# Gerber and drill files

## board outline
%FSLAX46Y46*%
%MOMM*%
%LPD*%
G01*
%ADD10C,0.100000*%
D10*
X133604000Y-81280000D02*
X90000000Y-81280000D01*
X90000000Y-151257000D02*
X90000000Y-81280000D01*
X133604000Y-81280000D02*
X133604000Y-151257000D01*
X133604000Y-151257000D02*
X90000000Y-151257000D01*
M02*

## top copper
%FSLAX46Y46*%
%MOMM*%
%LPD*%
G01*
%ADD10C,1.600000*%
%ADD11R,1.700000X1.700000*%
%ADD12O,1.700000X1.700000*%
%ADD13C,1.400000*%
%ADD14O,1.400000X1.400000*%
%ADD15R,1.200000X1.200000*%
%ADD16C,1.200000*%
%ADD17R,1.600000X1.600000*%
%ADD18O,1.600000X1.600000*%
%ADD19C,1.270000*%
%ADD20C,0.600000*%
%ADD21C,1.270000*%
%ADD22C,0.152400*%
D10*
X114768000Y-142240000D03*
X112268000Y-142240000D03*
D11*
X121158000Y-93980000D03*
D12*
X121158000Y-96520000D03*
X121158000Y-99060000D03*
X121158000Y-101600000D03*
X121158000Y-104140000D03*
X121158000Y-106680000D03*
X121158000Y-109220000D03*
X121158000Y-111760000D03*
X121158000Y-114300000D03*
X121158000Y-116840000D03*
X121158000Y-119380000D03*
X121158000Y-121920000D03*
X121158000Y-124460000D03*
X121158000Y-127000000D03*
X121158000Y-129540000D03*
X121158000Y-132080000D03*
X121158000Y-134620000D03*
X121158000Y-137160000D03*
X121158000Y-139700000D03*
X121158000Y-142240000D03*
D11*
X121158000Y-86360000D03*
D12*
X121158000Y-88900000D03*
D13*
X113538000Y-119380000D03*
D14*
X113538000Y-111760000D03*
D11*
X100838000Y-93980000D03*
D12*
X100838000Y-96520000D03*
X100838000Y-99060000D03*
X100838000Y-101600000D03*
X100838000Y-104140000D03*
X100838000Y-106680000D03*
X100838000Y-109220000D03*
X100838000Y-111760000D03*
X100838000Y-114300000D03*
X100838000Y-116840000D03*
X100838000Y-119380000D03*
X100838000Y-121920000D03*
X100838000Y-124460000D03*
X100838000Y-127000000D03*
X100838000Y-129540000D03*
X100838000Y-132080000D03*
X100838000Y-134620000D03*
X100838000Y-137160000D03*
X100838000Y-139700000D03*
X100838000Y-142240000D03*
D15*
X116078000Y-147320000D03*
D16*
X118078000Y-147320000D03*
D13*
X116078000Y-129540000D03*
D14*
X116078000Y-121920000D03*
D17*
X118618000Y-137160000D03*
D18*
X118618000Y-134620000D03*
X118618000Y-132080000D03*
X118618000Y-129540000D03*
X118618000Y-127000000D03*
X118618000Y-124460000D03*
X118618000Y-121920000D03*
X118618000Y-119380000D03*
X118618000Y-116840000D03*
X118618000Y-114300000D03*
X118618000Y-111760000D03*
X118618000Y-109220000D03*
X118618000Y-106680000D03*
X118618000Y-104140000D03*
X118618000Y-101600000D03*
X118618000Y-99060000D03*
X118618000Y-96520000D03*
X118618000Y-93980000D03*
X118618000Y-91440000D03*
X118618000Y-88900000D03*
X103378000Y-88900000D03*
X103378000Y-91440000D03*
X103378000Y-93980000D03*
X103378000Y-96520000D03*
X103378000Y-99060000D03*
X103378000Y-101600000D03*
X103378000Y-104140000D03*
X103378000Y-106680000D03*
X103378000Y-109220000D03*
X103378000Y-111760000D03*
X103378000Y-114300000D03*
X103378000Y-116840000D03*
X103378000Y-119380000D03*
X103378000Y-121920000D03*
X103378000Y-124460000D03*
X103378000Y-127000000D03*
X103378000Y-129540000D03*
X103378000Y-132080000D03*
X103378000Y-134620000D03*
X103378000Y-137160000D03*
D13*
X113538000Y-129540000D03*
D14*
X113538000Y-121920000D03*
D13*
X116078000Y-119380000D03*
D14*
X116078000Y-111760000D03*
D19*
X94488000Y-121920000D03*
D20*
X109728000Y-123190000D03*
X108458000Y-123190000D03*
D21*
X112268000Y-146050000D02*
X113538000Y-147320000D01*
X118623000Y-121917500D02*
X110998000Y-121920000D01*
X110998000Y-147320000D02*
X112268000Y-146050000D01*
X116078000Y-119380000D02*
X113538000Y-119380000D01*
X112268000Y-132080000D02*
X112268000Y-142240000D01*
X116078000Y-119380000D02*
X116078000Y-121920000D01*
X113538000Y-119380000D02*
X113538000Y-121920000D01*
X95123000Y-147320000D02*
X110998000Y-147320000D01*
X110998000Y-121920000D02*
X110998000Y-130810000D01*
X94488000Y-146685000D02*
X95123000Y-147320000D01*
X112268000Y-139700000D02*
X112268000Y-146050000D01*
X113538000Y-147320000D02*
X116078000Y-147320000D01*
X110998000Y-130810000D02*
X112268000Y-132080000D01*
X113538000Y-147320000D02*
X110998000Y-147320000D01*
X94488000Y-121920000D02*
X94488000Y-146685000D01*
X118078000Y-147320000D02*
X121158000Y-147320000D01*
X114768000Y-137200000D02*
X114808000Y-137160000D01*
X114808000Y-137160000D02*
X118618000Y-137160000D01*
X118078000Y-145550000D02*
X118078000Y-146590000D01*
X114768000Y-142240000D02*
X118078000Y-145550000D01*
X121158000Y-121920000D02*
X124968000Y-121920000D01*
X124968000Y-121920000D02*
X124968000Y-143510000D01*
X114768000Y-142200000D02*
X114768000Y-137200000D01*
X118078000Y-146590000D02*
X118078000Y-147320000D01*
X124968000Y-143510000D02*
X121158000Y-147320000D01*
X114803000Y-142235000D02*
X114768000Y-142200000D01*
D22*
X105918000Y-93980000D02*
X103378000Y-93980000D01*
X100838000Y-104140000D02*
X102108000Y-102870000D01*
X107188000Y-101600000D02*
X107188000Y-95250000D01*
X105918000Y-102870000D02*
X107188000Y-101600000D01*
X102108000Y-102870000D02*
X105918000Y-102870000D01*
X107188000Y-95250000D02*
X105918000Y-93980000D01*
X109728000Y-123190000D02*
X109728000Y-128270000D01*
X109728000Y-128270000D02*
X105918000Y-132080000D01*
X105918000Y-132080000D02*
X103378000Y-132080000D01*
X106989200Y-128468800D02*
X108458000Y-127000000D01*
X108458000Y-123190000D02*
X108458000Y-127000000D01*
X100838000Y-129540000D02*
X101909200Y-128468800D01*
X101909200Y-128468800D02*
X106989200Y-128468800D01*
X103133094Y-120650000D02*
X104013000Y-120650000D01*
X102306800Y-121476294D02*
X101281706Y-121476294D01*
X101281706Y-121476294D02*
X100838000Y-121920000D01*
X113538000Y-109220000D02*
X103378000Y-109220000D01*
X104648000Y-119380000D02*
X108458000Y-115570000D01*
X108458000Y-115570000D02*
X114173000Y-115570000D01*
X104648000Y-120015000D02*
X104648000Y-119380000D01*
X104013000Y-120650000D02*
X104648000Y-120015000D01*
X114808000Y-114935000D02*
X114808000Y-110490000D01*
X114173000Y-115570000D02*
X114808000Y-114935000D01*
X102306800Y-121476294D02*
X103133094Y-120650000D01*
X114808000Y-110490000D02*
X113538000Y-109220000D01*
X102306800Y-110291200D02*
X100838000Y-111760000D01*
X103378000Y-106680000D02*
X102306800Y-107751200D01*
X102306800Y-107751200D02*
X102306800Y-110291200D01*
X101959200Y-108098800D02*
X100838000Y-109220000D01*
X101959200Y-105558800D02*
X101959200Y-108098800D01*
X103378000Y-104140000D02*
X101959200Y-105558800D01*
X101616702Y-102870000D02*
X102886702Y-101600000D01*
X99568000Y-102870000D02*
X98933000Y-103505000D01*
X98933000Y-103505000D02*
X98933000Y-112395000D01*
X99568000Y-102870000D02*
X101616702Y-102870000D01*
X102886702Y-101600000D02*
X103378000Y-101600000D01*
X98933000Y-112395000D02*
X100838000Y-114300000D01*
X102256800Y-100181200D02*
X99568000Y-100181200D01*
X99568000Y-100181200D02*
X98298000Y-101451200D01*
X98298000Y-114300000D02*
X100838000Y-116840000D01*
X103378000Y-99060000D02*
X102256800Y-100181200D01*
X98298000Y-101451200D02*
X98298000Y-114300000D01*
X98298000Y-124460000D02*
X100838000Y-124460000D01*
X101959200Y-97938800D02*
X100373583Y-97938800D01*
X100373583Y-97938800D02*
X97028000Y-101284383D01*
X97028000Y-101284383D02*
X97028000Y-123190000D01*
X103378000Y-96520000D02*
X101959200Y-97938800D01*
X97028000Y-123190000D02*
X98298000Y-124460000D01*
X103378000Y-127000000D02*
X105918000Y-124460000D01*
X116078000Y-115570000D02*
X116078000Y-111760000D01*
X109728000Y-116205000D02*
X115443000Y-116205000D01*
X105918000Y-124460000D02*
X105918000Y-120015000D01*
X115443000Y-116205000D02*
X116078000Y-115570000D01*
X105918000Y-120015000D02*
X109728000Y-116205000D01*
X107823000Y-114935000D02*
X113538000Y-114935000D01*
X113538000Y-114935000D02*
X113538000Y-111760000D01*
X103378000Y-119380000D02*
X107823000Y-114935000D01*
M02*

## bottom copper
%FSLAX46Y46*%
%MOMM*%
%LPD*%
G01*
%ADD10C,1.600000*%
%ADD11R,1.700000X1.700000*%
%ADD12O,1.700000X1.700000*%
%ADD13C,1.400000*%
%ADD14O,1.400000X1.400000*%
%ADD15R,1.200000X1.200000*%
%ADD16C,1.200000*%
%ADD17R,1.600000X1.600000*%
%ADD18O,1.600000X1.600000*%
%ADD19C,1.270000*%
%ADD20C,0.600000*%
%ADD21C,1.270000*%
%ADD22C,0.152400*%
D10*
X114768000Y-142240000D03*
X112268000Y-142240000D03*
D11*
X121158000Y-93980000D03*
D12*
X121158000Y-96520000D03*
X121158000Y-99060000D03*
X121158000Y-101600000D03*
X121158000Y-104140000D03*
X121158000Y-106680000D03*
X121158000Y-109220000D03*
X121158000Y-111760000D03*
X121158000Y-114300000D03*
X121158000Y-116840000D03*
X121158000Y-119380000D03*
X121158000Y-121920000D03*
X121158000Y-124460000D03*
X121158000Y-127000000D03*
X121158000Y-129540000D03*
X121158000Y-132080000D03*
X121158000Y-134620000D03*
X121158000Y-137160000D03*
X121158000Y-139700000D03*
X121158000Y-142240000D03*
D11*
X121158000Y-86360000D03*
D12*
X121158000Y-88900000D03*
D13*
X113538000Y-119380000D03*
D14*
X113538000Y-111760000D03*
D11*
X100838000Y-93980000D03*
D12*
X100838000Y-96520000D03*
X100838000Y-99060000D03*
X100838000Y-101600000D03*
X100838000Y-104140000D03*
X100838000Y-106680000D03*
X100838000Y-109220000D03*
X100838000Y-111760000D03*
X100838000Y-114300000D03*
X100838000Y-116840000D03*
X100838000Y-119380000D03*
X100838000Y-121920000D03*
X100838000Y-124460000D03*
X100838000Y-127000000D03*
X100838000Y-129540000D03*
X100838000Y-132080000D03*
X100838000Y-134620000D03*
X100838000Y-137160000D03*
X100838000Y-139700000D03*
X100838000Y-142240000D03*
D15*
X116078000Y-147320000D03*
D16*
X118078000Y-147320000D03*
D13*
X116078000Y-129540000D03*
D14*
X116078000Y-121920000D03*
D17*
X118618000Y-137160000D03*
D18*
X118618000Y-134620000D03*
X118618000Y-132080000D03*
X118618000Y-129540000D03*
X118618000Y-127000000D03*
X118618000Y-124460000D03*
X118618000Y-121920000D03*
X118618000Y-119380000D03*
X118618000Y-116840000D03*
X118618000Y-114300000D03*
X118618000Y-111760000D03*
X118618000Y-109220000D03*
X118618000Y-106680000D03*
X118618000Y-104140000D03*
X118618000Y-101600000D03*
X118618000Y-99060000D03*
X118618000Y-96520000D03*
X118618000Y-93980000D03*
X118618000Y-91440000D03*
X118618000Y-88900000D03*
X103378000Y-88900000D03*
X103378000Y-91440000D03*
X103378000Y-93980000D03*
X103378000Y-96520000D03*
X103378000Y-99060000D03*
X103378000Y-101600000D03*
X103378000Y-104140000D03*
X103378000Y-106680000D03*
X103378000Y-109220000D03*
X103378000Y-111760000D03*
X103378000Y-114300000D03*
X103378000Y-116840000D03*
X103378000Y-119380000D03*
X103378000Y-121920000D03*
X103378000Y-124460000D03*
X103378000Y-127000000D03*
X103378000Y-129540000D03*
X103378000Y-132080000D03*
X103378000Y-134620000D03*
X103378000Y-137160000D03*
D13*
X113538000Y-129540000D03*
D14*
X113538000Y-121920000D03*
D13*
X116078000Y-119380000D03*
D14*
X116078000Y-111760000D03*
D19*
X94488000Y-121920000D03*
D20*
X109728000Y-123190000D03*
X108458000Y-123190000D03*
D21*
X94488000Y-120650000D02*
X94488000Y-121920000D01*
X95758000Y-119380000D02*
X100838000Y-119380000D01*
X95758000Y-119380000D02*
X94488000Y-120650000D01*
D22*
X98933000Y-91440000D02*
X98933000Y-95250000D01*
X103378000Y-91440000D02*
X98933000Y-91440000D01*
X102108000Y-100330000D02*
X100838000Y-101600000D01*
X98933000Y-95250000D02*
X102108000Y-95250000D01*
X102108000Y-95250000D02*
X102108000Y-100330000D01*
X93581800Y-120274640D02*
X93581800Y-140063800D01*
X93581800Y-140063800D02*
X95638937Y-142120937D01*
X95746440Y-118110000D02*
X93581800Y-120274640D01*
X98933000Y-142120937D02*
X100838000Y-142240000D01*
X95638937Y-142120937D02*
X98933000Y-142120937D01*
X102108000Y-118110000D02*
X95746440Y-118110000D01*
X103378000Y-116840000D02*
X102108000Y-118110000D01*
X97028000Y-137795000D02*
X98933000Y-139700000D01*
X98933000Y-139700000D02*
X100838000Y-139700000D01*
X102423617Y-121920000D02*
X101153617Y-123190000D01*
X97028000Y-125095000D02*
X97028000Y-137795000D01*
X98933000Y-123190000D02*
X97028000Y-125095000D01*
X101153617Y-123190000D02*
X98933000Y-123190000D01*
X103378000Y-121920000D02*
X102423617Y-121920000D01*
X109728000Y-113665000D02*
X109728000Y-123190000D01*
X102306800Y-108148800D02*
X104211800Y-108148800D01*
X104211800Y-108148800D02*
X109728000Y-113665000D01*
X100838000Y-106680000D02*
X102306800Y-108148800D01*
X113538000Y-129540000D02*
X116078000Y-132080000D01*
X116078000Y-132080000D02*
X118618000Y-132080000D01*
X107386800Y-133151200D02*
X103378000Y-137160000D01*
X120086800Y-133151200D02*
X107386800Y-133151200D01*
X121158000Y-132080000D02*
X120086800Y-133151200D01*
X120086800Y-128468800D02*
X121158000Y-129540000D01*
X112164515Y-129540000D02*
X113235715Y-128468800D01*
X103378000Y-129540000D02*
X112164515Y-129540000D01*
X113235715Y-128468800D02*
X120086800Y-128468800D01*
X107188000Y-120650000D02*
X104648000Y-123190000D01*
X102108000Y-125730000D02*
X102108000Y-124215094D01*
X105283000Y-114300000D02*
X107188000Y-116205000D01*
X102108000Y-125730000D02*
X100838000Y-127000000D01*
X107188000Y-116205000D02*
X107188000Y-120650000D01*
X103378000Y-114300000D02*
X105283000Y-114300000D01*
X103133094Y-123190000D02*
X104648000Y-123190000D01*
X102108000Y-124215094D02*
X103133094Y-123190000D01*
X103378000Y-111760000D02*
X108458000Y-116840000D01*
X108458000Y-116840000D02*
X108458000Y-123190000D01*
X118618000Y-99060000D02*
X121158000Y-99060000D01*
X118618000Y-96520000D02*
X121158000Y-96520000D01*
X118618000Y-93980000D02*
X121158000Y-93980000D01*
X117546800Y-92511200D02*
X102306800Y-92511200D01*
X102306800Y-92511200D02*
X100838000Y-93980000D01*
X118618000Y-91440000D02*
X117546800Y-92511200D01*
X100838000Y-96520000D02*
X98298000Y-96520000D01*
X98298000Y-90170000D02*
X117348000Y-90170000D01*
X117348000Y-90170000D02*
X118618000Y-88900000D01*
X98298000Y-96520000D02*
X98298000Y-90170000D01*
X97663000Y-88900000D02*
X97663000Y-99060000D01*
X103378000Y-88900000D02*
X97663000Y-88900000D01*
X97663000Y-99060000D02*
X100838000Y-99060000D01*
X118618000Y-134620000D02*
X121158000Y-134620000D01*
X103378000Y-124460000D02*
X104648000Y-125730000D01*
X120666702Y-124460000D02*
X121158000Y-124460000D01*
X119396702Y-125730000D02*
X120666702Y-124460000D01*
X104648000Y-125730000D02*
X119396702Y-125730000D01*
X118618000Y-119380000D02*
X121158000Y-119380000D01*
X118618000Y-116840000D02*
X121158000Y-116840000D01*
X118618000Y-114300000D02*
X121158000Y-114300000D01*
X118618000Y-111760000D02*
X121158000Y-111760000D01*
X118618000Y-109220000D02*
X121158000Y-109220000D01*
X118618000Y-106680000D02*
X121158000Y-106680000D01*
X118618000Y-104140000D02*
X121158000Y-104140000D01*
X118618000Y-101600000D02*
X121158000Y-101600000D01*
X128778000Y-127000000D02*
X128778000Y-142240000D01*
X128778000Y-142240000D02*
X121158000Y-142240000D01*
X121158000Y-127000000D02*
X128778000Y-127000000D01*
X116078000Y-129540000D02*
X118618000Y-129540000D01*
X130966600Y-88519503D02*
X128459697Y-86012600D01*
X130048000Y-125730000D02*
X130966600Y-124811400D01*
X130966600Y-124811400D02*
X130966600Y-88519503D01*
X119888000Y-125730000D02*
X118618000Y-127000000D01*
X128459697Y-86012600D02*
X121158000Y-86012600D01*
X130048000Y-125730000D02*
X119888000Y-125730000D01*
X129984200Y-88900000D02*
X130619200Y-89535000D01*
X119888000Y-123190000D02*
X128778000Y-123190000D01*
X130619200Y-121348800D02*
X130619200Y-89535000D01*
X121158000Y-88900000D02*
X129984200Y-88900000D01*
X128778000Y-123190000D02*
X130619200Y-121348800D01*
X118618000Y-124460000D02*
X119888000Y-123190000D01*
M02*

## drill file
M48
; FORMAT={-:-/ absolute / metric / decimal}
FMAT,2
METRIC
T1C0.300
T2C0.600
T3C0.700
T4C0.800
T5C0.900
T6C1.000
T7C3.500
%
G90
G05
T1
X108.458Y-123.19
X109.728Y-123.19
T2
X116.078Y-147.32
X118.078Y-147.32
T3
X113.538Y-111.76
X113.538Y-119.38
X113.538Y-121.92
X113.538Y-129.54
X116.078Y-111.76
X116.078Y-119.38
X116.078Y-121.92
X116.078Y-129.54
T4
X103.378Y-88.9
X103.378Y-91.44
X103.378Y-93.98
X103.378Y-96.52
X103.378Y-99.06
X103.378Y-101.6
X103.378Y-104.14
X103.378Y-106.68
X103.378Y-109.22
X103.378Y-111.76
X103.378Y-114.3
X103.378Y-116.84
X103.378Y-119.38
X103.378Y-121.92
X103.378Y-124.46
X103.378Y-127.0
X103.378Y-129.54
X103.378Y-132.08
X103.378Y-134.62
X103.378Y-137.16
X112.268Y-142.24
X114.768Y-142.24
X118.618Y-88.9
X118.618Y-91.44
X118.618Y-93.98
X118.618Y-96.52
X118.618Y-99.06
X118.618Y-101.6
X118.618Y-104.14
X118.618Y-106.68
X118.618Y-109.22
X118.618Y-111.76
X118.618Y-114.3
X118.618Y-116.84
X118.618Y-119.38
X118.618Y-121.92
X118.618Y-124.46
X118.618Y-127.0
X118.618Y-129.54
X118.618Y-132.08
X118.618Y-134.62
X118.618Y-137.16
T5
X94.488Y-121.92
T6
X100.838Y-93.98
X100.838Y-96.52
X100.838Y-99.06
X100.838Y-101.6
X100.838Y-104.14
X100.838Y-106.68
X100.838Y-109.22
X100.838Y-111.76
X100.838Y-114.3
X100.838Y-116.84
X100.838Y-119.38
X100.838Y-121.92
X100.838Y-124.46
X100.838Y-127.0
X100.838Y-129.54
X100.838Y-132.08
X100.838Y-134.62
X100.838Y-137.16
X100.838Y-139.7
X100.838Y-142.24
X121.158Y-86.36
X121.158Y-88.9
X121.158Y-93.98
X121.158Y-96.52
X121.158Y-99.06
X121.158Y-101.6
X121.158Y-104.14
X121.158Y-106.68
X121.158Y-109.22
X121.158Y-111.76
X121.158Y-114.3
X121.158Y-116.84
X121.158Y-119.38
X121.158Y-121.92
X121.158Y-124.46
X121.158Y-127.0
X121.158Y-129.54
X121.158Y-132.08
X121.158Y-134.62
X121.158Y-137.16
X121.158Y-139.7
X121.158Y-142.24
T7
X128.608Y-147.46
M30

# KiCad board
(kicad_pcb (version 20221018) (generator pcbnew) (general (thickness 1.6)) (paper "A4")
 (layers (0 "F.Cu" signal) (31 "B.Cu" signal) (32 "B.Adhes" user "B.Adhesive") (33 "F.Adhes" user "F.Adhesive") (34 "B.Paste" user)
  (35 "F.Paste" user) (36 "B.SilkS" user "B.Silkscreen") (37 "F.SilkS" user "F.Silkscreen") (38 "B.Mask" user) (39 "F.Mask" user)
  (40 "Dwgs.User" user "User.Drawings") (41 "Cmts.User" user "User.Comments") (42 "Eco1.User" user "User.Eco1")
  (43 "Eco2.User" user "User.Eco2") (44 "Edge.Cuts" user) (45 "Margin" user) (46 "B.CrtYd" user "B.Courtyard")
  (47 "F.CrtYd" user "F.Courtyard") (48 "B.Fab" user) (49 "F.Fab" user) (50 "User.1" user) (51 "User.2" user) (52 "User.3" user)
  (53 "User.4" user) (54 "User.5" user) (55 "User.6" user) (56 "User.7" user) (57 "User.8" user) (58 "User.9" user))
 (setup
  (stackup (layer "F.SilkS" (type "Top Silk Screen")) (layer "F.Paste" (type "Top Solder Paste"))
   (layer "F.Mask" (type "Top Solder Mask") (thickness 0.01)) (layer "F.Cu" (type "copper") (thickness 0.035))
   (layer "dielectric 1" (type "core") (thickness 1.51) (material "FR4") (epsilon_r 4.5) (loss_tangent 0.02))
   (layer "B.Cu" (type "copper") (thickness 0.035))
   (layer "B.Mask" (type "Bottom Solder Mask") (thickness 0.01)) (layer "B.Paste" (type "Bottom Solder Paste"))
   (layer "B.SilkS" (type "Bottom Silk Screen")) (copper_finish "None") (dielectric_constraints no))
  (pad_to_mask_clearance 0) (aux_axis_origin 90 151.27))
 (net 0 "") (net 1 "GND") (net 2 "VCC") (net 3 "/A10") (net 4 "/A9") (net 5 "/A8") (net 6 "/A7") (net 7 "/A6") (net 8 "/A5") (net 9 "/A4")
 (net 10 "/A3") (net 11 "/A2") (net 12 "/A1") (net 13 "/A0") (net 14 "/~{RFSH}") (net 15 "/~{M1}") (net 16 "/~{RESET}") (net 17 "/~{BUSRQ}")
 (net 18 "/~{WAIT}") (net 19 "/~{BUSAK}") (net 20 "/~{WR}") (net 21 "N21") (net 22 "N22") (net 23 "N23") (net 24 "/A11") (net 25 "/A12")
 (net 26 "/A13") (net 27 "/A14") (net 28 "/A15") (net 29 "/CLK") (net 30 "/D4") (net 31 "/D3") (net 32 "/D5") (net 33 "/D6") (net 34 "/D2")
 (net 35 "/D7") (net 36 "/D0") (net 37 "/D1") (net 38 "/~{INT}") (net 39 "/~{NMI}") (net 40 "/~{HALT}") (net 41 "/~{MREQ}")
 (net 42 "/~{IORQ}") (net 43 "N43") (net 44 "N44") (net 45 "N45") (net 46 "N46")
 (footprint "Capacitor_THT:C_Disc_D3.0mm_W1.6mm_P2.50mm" (layer "F.Cu") (at 114.768 142.24 180)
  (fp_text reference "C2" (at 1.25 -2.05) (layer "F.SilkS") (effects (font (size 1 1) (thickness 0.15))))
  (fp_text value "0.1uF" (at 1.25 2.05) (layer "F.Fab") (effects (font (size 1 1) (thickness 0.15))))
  (pad "1" thru_hole circle (at 0 0 180) (size 1.6 1.6) (drill 0.8) (layers "*.Cu" "*.Mask") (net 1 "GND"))
  (pad "2" thru_hole circle (at 2.5 0 180) (size 1.6 1.6) (drill 0.8) (layers "*.Cu" "*.Mask") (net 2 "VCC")))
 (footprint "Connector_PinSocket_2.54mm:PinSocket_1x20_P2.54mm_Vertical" (layer "F.Cu") (at 121.158 93.98)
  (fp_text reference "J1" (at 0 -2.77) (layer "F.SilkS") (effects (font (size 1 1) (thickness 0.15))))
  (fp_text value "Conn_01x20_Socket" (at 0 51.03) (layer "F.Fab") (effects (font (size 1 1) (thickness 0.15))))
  (pad "1" thru_hole rect (at 0 0) (size 1.7 1.7) (drill 1) (layers "*.Cu" "*.Mask") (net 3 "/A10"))
  (pad "2" thru_hole oval (at 0 2.54) (size 1.7 1.7) (drill 1) (layers "*.Cu" "*.Mask") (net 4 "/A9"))
  (pad "3" thru_hole oval (at 0 5.08) (size 1.7 1.7) (drill 1) (layers "*.Cu" "*.Mask") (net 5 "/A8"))
  (pad "4" thru_hole oval (at 0 7.62) (size 1.7 1.7) (drill 1) (layers "*.Cu" "*.Mask") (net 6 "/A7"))
  (pad "5" thru_hole oval (at 0 10.16) (size 1.7 1.7) (drill 1) (layers "*.Cu" "*.Mask") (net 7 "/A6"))
  (pad "6" thru_hole oval (at 0 12.7) (size 1.7 1.7) (drill 1) (layers "*.Cu" "*.Mask") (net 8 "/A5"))
  (pad "7" thru_hole oval (at 0 15.24) (size 1.7 1.7) (drill 1) (layers "*.Cu" "*.Mask") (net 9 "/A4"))
  (pad "8" thru_hole oval (at 0 17.78) (size 1.7 1.7) (drill 1) (layers "*.Cu" "*.Mask") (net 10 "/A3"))
  (pad "9" thru_hole oval (at 0 20.32) (size 1.7 1.7) (drill 1) (layers "*.Cu" "*.Mask") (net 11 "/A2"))
  (pad "10" thru_hole oval (at 0 22.86) (size 1.7 1.7) (drill 1) (layers "*.Cu" "*.Mask") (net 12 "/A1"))
  (pad "11" thru_hole oval (at 0 25.4) (size 1.7 1.7) (drill 1) (layers "*.Cu" "*.Mask") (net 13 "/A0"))
  (pad "12" thru_hole oval (at 0 27.94) (size 1.7 1.7) (drill 1) (layers "*.Cu" "*.Mask") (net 1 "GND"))
  (pad "13" thru_hole oval (at 0 30.48) (size 1.7 1.7) (drill 1) (layers "*.Cu" "*.Mask") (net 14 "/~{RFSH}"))
  (pad "14" thru_hole oval (at 0 33.02) (size 1.7 1.7) (drill 1) (layers "*.Cu" "*.Mask") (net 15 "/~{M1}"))
  (pad "15" thru_hole oval (at 0 35.56) (size 1.7 1.7) (drill 1) (layers "*.Cu" "*.Mask") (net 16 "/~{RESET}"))
  (pad "16" thru_hole oval (at 0 38.1) (size 1.7 1.7) (drill 1) (layers "*.Cu" "*.Mask") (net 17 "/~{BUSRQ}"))
  (pad "17" thru_hole oval (at 0 40.64) (size 1.7 1.7) (drill 1) (layers "*.Cu" "*.Mask") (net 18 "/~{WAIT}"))
  (pad "18" thru_hole oval (at 0 43.18) (size 1.7 1.7) (drill 1) (layers "*.Cu" "*.Mask") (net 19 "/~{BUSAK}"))
  (pad "19" thru_hole oval (at 0 45.72) (size 1.7 1.7) (drill 1) (layers "*.Cu" "*.Mask") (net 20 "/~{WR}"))
  (pad "20" thru_hole oval (at 0 48.26) (size 1.7 1.7) (drill 1) (layers "*.Cu" "*.Mask") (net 15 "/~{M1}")))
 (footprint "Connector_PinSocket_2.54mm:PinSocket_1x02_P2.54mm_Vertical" (layer "F.Cu") (at 121.158 86.36)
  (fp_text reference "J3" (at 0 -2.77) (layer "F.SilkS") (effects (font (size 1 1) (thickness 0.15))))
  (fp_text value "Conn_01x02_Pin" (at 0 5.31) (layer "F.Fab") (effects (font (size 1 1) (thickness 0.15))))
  (pad "1" thru_hole rect (at 0 0) (size 1.7 1.7) (drill 1) (layers "*.Cu" "*.Mask") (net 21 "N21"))
  (pad "2" thru_hole oval (at 0 2.54) (size 1.7 1.7) (drill 1) (layers "*.Cu" "*.Mask") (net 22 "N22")))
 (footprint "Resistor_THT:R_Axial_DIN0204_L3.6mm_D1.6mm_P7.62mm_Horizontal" (layer "F.Cu") (at 113.538 119.38 90)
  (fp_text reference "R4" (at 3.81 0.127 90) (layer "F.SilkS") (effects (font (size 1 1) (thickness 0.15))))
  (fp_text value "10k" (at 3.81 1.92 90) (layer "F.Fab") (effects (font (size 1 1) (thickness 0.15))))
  (pad "1" thru_hole circle (at 0 0 90) (size 1.4 1.4) (drill 0.7) (layers "*.Cu" "*.Mask") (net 2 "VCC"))
  (pad "2" thru_hole oval (at 7.62 0 90) (size 1.4 1.4) (drill 0.7) (layers "*.Cu" "*.Mask") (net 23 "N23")))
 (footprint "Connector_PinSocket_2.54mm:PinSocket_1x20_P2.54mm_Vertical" (layer "F.Cu") (at 100.838 93.98)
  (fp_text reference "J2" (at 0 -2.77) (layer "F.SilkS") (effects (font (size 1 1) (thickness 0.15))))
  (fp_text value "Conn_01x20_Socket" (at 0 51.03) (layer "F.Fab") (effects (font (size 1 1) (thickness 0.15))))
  (pad "1" thru_hole rect (at 0 0) (size 1.7 1.7) (drill 1) (layers "*.Cu" "*.Mask") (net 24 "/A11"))
  (pad "2" thru_hole oval (at 0 2.54) (size 1.7 1.7) (drill 1) (layers "*.Cu" "*.Mask") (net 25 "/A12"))
  (pad "3" thru_hole oval (at 0 5.08) (size 1.7 1.7) (drill 1) (layers "*.Cu" "*.Mask") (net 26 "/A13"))
  (pad "4" thru_hole oval (at 0 7.62) (size 1.7 1.7) (drill 1) (layers "*.Cu" "*.Mask") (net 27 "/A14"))
  (pad "5" thru_hole oval (at 0 10.16) (size 1.7 1.7) (drill 1) (layers "*.Cu" "*.Mask") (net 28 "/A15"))
  (pad "6" thru_hole oval (at 0 12.7) (size 1.7 1.7) (drill 1) (layers "*.Cu" "*.Mask") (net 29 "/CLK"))
  (pad "7" thru_hole oval (at 0 15.24) (size 1.7 1.7) (drill 1) (layers "*.Cu" "*.Mask") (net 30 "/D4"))
  (pad "8" thru_hole oval (at 0 17.78) (size 1.7 1.7) (drill 1) (layers "*.Cu" "*.Mask") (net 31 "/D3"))
  (pad "9" thru_hole oval (at 0 20.32) (size 1.7 1.7) (drill 1) (layers "*.Cu" "*.Mask") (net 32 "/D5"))
  (pad "10" thru_hole oval (at 0 22.86) (size 1.7 1.7) (drill 1) (layers "*.Cu" "*.Mask") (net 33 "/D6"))
  (pad "11" thru_hole oval (at 0 25.4) (size 1.7 1.7) (drill 1) (layers "*.Cu" "*.Mask") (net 2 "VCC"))
  (pad "12" thru_hole oval (at 0 27.94) (size 1.7 1.7) (drill 1) (layers "*.Cu" "*.Mask") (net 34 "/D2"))
  (pad "13" thru_hole oval (at 0 30.48) (size 1.7 1.7) (drill 1) (layers "*.Cu" "*.Mask") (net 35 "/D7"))
  (pad "14" thru_hole oval (at 0 33.02) (size 1.7 1.7) (drill 1) (layers "*.Cu" "*.Mask") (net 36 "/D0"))
  (pad "15" thru_hole oval (at 0 35.56) (size 1.7 1.7) (drill 1) (layers "*.Cu" "*.Mask") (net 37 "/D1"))
  (pad "16" thru_hole oval (at 0 38.1) (size 1.7 1.7) (drill 1) (layers "*.Cu" "*.Mask") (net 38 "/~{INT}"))
  (pad "17" thru_hole oval (at 0 40.64) (size 1.7 1.7) (drill 1) (layers "*.Cu" "*.Mask") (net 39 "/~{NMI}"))
  (pad "18" thru_hole oval (at 0 43.18) (size 1.7 1.7) (drill 1) (layers "*.Cu" "*.Mask") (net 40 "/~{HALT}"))
  (pad "19" thru_hole oval (at 0 45.72) (size 1.7 1.7) (drill 1) (layers "*.Cu" "*.Mask") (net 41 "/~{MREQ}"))
  (pad "20" thru_hole oval (at 0 48.26) (size 1.7 1.7) (drill 1) (layers "*.Cu" "*.Mask") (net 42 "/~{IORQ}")))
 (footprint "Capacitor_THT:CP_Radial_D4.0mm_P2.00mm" (layer "F.Cu") (at 116.078 147.32)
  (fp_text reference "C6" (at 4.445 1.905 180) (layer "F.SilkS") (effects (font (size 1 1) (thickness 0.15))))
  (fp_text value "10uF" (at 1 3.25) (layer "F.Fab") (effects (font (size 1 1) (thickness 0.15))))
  (pad "1" thru_hole rect (at 0 0) (size 1.2 1.2) (drill 0.6) (layers "*.Cu" "*.Mask") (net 2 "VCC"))
  (pad "2" thru_hole circle (at 2 0) (size 1.2 1.2) (drill 0.6) (layers "*.Cu" "*.Mask") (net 1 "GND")))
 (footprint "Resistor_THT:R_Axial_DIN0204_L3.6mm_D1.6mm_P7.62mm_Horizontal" (layer "F.Cu") (at 116.078 129.54 90)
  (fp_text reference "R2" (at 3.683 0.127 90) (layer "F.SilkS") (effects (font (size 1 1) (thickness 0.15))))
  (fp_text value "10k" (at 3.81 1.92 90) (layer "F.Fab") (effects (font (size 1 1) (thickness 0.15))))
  (pad "1" thru_hole circle (at 0 0 90) (size 1.4 1.4) (drill 0.7) (layers "*.Cu" "*.Mask") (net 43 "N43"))
  (pad "2" thru_hole oval (at 7.62 0 90) (size 1.4 1.4) (drill 0.7) (layers "*.Cu" "*.Mask") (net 2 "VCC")))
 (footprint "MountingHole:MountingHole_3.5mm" (layer "F.Cu") (at 128.608 147.46)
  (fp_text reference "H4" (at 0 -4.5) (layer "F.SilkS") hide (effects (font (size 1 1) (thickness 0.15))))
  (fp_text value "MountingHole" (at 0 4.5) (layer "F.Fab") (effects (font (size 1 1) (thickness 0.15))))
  (pad "" np_thru_hole circle (at 0 0) (size 3.5 3.5) (drill 3.5) (layers "*.Cu" "*.Mask")))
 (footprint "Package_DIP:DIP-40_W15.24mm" (layer "F.Cu") (at 118.618 137.16 180)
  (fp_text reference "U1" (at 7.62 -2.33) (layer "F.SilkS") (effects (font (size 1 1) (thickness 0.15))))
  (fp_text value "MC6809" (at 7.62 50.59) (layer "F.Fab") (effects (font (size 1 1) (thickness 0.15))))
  (pad "1" thru_hole rect (at 0 0 180) (size 1.6 1.6) (drill 0.8) (layers "*.Cu" "*.Mask") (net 1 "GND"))
  (pad "2" thru_hole oval (at 0 2.54 180) (size 1.6 1.6) (drill 0.8) (layers "*.Cu" "*.Mask") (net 18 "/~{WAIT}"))
  (pad "3" thru_hole oval (at 0 5.08 180) (size 1.6 1.6) (drill 0.8) (layers "*.Cu" "*.Mask") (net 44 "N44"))
  (pad "4" thru_hole oval (at 0 7.62 180) (size 1.6 1.6) (drill 0.8) (layers "*.Cu" "*.Mask") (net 43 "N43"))
  (pad "5" thru_hole oval (at 0 10.16 180) (size 1.6 1.6) (drill 0.8) (layers "*.Cu" "*.Mask") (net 21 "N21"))
  (pad "6" thru_hole oval (at 0 12.7 180) (size 1.6 1.6) (drill 0.8) (layers "*.Cu" "*.Mask") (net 22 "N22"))
  (pad "7" thru_hole oval (at 0 15.24 180) (size 1.6 1.6) (drill 0.8) (layers "*.Cu" "*.Mask") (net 2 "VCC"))
  (pad "8" thru_hole oval (at 0 17.78 180) (size 1.6 1.6) (drill 0.8) (layers "*.Cu" "*.Mask") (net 13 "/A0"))
  (pad "9" thru_hole oval (at 0 20.32 180) (size 1.6 1.6) (drill 0.8) (layers "*.Cu" "*.Mask") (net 12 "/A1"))
  (pad "10" thru_hole oval (at 0 22.86 180) (size 1.6 1.6) (drill 0.8) (layers "*.Cu" "*.Mask") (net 11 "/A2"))
  (pad "11" thru_hole oval (at 0 25.4 180) (size 1.6 1.6) (drill 0.8) (layers "*.Cu" "*.Mask") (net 10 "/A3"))
  (pad "12" thru_hole oval (at 0 27.94 180) (size 1.6 1.6) (drill 0.8) (layers "*.Cu" "*.Mask") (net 9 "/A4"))
  (pad "13" thru_hole oval (at 0 30.48 180) (size 1.6 1.6) (drill 0.8) (layers "*.Cu" "*.Mask") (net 8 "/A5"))
  (pad "14" thru_hole oval (at 0 33.02 180) (size 1.6 1.6) (drill 0.8) (layers "*.Cu" "*.Mask") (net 7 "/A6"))
  (pad "15" thru_hole oval (at 0 35.56 180) (size 1.6 1.6) (drill 0.8) (layers "*.Cu" "*.Mask") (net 6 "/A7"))
  (pad "16" thru_hole oval (at 0 38.1 180) (size 1.6 1.6) (drill 0.8) (layers "*.Cu" "*.Mask") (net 5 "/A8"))
  (pad "17" thru_hole oval (at 0 40.64 180) (size 1.6 1.6) (drill 0.8) (layers "*.Cu" "*.Mask") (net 4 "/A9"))
  (pad "18" thru_hole oval (at 0 43.18 180) (size 1.6 1.6) (drill 0.8) (layers "*.Cu" "*.Mask") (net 3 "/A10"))
  (pad "19" thru_hole oval (at 0 45.72 180) (size 1.6 1.6) (drill 0.8) (layers "*.Cu" "*.Mask") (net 24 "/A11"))
  (pad "20" thru_hole oval (at 0 48.26 180) (size 1.6 1.6) (drill 0.8) (layers "*.Cu" "*.Mask") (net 25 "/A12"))
  (pad "21" thru_hole oval (at 15.24 48.26 180) (size 1.6 1.6) (drill 0.8) (layers "*.Cu" "*.Mask") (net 26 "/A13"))
  (pad "22" thru_hole oval (at 15.24 45.72 180) (size 1.6 1.6) (drill 0.8) (layers "*.Cu" "*.Mask") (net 27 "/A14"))
  (pad "23" thru_hole oval (at 15.24 43.18 180) (size 1.6 1.6) (drill 0.8) (layers "*.Cu" "*.Mask") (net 28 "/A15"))
  (pad "24" thru_hole oval (at 15.24 40.64 180) (size 1.6 1.6) (drill 0.8) (layers "*.Cu" "*.Mask") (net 35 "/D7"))
  (pad "25" thru_hole oval (at 15.24 38.1 180) (size 1.6 1.6) (drill 0.8) (layers "*.Cu" "*.Mask") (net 33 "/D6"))
  (pad "26" thru_hole oval (at 15.24 35.56 180) (size 1.6 1.6) (drill 0.8) (layers "*.Cu" "*.Mask") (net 32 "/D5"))
  (pad "27" thru_hole oval (at 15.24 33.02 180) (size 1.6 1.6) (drill 0.8) (layers "*.Cu" "*.Mask") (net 30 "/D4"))
  (pad "28" thru_hole oval (at 15.24 30.48 180) (size 1.6 1.6) (drill 0.8) (layers "*.Cu" "*.Mask") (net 31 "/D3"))
  (pad "29" thru_hole oval (at 15.24 27.94 180) (size 1.6 1.6) (drill 0.8) (layers "*.Cu" "*.Mask") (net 34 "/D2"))
  (pad "30" thru_hole oval (at 15.24 25.4 180) (size 1.6 1.6) (drill 0.8) (layers "*.Cu" "*.Mask") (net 37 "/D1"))
  (pad "31" thru_hole oval (at 15.24 22.86 180) (size 1.6 1.6) (drill 0.8) (layers "*.Cu" "*.Mask") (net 36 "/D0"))
  (pad "32" thru_hole oval (at 15.24 20.32 180) (size 1.6 1.6) (drill 0.8) (layers "*.Cu" "*.Mask") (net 42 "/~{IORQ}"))
  (pad "33" thru_hole oval (at 15.24 17.78 180) (size 1.6 1.6) (drill 0.8) (layers "*.Cu" "*.Mask") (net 23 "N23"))
  (pad "34" thru_hole oval (at 15.24 15.24 180) (size 1.6 1.6) (drill 0.8) (layers "*.Cu" "*.Mask") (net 41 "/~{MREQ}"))
  (pad "35" thru_hole oval (at 15.24 12.7 180) (size 1.6 1.6) (drill 0.8) (layers "*.Cu" "*.Mask") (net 14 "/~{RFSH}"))
  (pad "36" thru_hole oval (at 15.24 10.16 180) (size 1.6 1.6) (drill 0.8) (layers "*.Cu" "*.Mask") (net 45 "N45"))
  (pad "37" thru_hole oval (at 15.24 7.62 180) (size 1.6 1.6) (drill 0.8) (layers "*.Cu" "*.Mask") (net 16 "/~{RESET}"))
  (pad "38" thru_hole oval (at 15.24 5.08 180) (size 1.6 1.6) (drill 0.8) (layers "*.Cu" "*.Mask") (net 29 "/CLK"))
  (pad "39" thru_hole oval (at 15.24 2.54 180) (size 1.6 1.6) (drill 0.8) (layers "*.Cu" "*.Mask") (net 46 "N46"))
  (pad "40" thru_hole oval (at 15.24 0 180) (size 1.6 1.6) (drill 0.8) (layers "*.Cu" "*.Mask") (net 17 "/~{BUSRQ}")))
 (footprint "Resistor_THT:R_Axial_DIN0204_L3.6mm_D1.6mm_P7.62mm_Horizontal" (layer "F.Cu") (at 113.538 129.54 90)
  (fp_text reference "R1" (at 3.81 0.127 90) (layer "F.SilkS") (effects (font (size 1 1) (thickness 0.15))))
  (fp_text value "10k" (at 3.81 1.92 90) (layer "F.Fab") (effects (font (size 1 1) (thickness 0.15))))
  (pad "1" thru_hole circle (at 0 0 90) (size 1.4 1.4) (drill 0.7) (layers "*.Cu" "*.Mask") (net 44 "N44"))
  (pad "2" thru_hole oval (at 7.62 0 90) (size 1.4 1.4) (drill 0.7) (layers "*.Cu" "*.Mask") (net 2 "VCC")))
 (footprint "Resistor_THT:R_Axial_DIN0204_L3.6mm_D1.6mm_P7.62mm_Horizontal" (layer "F.Cu") (at 116.078 119.38 90)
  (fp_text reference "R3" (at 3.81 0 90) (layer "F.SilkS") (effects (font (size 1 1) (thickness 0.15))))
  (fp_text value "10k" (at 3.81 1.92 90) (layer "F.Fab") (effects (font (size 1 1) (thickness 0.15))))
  (pad "1" thru_hole circle (at 0 0 90) (size 1.4 1.4) (drill 0.7) (layers "*.Cu" "*.Mask") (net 2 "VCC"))
  (pad "2" thru_hole oval (at 7.62 0 90) (size 1.4 1.4) (drill 0.7) (layers "*.Cu" "*.Mask") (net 45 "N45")))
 (gr_line (start 133.604 81.28) (end 90 81.28) (stroke (width 0.1) (type solid)) (layer "Edge.Cuts"))
 (gr_line (start 90 151.257) (end 90 81.28) (stroke (width 0.1) (type solid)) (layer "Edge.Cuts"))
 (gr_line (start 133.604 81.28) (end 133.604 151.257) (stroke (width 0.1) (type solid)) (layer "Edge.Cuts"))
 (gr_line (start 133.604 151.257) (end 90 151.257) (stroke (width 0.1) (type solid)) (layer "Edge.Cuts"))
 (segment (start 112.268 146.05) (end 113.538 147.32) (width 1.27) (layer "F.Cu") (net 2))
 (segment (start 118.623 121.9175) (end 110.998 121.92) (width 1.27) (layer "F.Cu") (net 2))
 (segment (start 110.998 147.32) (end 112.268 146.05) (width 1.27) (layer "F.Cu") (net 2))
 (segment (start 116.078 119.38) (end 113.538 119.38) (width 1.27) (layer "F.Cu") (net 2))
 (segment (start 112.268 132.08) (end 112.268 142.24) (width 1.27) (layer "F.Cu") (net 2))
 (segment (start 116.078 119.38) (end 116.078 121.92) (width 1.27) (layer "F.Cu") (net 2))
 (segment (start 113.538 119.38) (end 113.538 121.92) (width 1.27) (layer "F.Cu") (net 2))
 (segment (start 95.123 147.32) (end 110.998 147.32) (width 1.27) (layer "F.Cu") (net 2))
 (segment (start 110.998 121.92) (end 110.998 130.81) (width 1.27) (layer "F.Cu") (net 2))
 (segment (start 94.488 146.685) (end 95.123 147.32) (width 1.27) (layer "F.Cu") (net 2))
 (segment (start 112.268 139.7) (end 112.268 146.05) (width 1.27) (layer "F.Cu") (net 2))
 (segment (start 113.538 147.32) (end 116.078 147.32) (width 1.27) (layer "F.Cu") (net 2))
 (segment (start 110.998 130.81) (end 112.268 132.08) (width 1.27) (layer "F.Cu") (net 2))
 (segment (start 113.538 147.32) (end 110.998 147.32) (width 1.27) (layer "F.Cu") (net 2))
 (segment (start 94.488 121.92) (end 94.488 146.685) (width 1.27) (layer "F.Cu") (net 2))
 (via (at 94.488 121.92) (size 1.27) (drill 0.9) (layers "F.Cu" "B.Cu") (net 2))
 (segment (start 94.488 120.65) (end 94.488 121.92) (width 1.27) (layer "B.Cu") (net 2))
 (segment (start 95.758 119.38) (end 100.838 119.38) (width 1.27) (layer "B.Cu") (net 2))
 (segment (start 95.758 119.38) (end 94.488 120.65) (width 1.27) (layer "B.Cu") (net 2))
 (segment (start 98.933 91.44) (end 98.933 95.25) (width 0.1524) (layer "B.Cu") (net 27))
 (segment (start 103.378 91.44) (end 98.933 91.44) (width 0.1524) (layer "B.Cu") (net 27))
 (segment (start 102.108 100.33) (end 100.838 101.6) (width 0.1524) (layer "B.Cu") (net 27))
 (segment (start 98.933 95.25) (end 102.108 95.25) (width 0.1524) (layer "B.Cu") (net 27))
 (segment (start 102.108 95.25) (end 102.108 100.33) (width 0.1524) (layer "B.Cu") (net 27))
 (segment (start 118.078 147.32) (end 121.158 147.32) (width 1.27) (layer "F.Cu") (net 1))
 (segment (start 114.768 137.2) (end 114.808 137.16) (width 1.27) (layer "F.Cu") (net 1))
 (segment (start 114.808 137.16) (end 118.618 137.16) (width 1.27) (layer "F.Cu") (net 1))
 (segment (start 118.078 145.55) (end 118.078 146.59) (width 1.27) (layer "F.Cu") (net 1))
 (segment (start 114.768 142.24) (end 118.078 145.55) (width 1.27) (layer "F.Cu") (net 1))
 (segment (start 121.158 121.92) (end 124.968 121.92) (width 1.27) (layer "F.Cu") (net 1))
 (segment (start 124.968 121.92) (end 124.968 143.51) (width 1.27) (layer "F.Cu") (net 1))
 (segment (start 114.768 142.2) (end 114.768 137.2) (width 1.27) (layer "F.Cu") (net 1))
 (segment (start 118.078 146.59) (end 118.078 147.32) (width 1.27) (layer "F.Cu") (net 1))
 (segment (start 124.968 143.51) (end 121.158 147.32) (width 1.27) (layer "F.Cu") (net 1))
 (segment (start 114.803 142.235) (end 114.768 142.2) (width 1.27) (layer "F.Cu") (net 1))
 (segment (start 105.918 93.98) (end 103.378 93.98) (width 0.1524) (layer "F.Cu") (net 28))
 (segment (start 100.838 104.14) (end 102.108 102.87) (width 0.1524) (layer "F.Cu") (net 28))
 (segment (start 107.188 101.6) (end 107.188 95.25) (width 0.1524) (layer "F.Cu") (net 28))
 (segment (start 105.918 102.87) (end 107.188 101.6) (width 0.1524) (layer "F.Cu") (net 28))
 (segment (start 102.108 102.87) (end 105.918 102.87) (width 0.1524) (layer "F.Cu") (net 28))
 (segment (start 107.188 95.25) (end 105.918 93.98) (width 0.1524) (layer "F.Cu") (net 28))
 (segment (start 93.5818 120.27464) (end 93.5818 140.0638) (width 0.1524) (layer "B.Cu") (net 42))
 (segment (start 93.5818 140.0638) (end 95.638937 142.120937) (width 0.1524) (layer "B.Cu") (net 42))
 (segment (start 95.74644 118.11) (end 93.5818 120.27464) (width 0.1524) (layer "B.Cu") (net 42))
 (segment (start 98.933 142.120937) (end 100.838 142.24) (width 0.1524) (layer "B.Cu") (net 42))
 (segment (start 95.638937 142.120937) (end 98.933 142.120937) (width 0.1524) (layer "B.Cu") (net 42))
 (segment (start 102.108 118.11) (end 95.74644 118.11) (width 0.1524) (layer "B.Cu") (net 42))
 (segment (start 103.378 116.84) (end 102.108 118.11) (width 0.1524) (layer "B.Cu") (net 42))
 (segment (start 97.028 137.795) (end 98.933 139.7) (width 0.1524) (layer "B.Cu") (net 41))
 (segment (start 98.933 139.7) (end 100.838 139.7) (width 0.1524) (layer "B.Cu") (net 41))
 (segment (start 102.423617 121.92) (end 101.153617 123.19) (width 0.1524) (layer "B.Cu") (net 41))
 (segment (start 97.028 125.095) (end 97.028 137.795) (width 0.1524) (layer "B.Cu") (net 41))
 (segment (start 98.933 123.19) (end 97.028 125.095) (width 0.1524) (layer "B.Cu") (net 41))
 (segment (start 101.153617 123.19) (end 98.933 123.19) (width 0.1524) (layer "B.Cu") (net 41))
 (segment (start 103.378 121.92) (end 102.423617 121.92) (width 0.1524) (layer "B.Cu") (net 41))
 (segment (start 109.728 123.19) (end 109.728 128.27) (width 0.1524) (layer "F.Cu") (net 29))
 (segment (start 109.728 128.27) (end 105.918 132.08) (width 0.1524) (layer "F.Cu") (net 29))
 (segment (start 105.918 132.08) (end 103.378 132.08) (width 0.1524) (layer "F.Cu") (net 29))
 (via (at 109.728 123.19) (size 0.6) (drill 0.3) (layers "F.Cu" "B.Cu") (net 29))
 (segment (start 109.728 113.665) (end 109.728 123.19) (width 0.1524) (layer "B.Cu") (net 29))
 (segment (start 102.3068 108.1488) (end 104.2118 108.1488) (width 0.1524) (layer "B.Cu") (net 29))
 (segment (start 104.2118 108.1488) (end 109.728 113.665) (width 0.1524) (layer "B.Cu") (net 29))
 (segment (start 100.838 106.68) (end 102.3068 108.1488) (width 0.1524) (layer "B.Cu") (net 29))
 (segment (start 113.538 129.54) (end 116.078 132.08) (width 0.1524) (layer "B.Cu") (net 44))
 (segment (start 116.078 132.08) (end 118.618 132.08) (width 0.1524) (layer "B.Cu") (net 44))
 (segment (start 107.3868 133.1512) (end 103.378 137.16) (width 0.1524) (layer "B.Cu") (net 17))
 (segment (start 120.0868 133.1512) (end 107.3868 133.1512) (width 0.1524) (layer "B.Cu") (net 17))
 (segment (start 121.158 132.08) (end 120.0868 133.1512) (width 0.1524) (layer "B.Cu") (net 17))
 (segment (start 120.0868 128.4688) (end 121.158 129.54) (width 0.1524) (layer "B.Cu") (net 16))
 (segment (start 112.164515 129.54) (end 113.235715 128.4688) (width 0.1524) (layer "B.Cu") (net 16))
 (segment (start 103.378 129.54) (end 112.164515 129.54) (width 0.1524) (layer "B.Cu") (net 16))
 (segment (start 113.235715 128.4688) (end 120.0868 128.4688) (width 0.1524) (layer "B.Cu") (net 16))
 (segment (start 107.188 120.65) (end 104.648 123.19) (width 0.1524) (layer "B.Cu") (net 36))
 (segment (start 102.108 125.73) (end 102.108 124.215094) (width 0.1524) (layer "B.Cu") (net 36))
 (segment (start 105.283 114.3) (end 107.188 116.205) (width 0.1524) (layer "B.Cu") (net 36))
 (segment (start 102.108 125.73) (end 100.838 127) (width 0.1524) (layer "B.Cu") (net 36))
 (segment (start 107.188 116.205) (end 107.188 120.65) (width 0.1524) (layer "B.Cu") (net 36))
 (segment (start 103.378 114.3) (end 105.283 114.3) (width 0.1524) (layer "B.Cu") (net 36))
 (segment (start 103.133094 123.19) (end 104.648 123.19) (width 0.1524) (layer "B.Cu") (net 36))
 (segment (start 102.108 124.215094) (end 103.133094 123.19) (width 0.1524) (layer "B.Cu") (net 36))
 (segment (start 106.9892 128.4688) (end 108.458 127) (width 0.1524) (layer "F.Cu") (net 37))
 (segment (start 108.458 123.19) (end 108.458 127) (width 0.1524) (layer "F.Cu") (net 37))
 (segment (start 100.838 129.54) (end 101.9092 128.4688) (width 0.1524) (layer "F.Cu") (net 37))
 (segment (start 101.9092 128.4688) (end 106.9892 128.4688) (width 0.1524) (layer "F.Cu") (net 37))
 (via (at 108.458 123.19) (size 0.6) (drill 0.3) (layers "F.Cu" "B.Cu") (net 37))
 (segment (start 103.378 111.76) (end 108.458 116.84) (width 0.1524) (layer "B.Cu") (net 37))
 (segment (start 108.458 116.84) (end 108.458 123.19) (width 0.1524) (layer "B.Cu") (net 37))
 (segment (start 103.133094 120.65) (end 104.013 120.65) (width 0.1524) (layer "F.Cu") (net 34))
 (segment (start 102.3068 121.476294) (end 101.281706 121.476294) (width 0.1524) (layer "F.Cu") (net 34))
 (segment (start 101.281706 121.476294) (end 100.838 121.92) (width 0.1524) (layer "F.Cu") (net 34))
 (segment (start 113.538 109.22) (end 103.378 109.22) (width 0.1524) (layer "F.Cu") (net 34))
 (segment (start 104.648 119.38) (end 108.458 115.57) (width 0.1524) (layer "F.Cu") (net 34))
 (segment (start 108.458 115.57) (end 114.173 115.57) (width 0.1524) (layer "F.Cu") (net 34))
 (segment (start 104.648 120.015) (end 104.648 119.38) (width 0.1524) (layer "F.Cu") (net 34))
 (segment (start 104.013 120.65) (end 104.648 120.015) (width 0.1524) (layer "F.Cu") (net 34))
 (segment (start 114.808 114.935) (end 114.808 110.49) (width 0.1524) (layer "F.Cu") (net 34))
 (segment (start 114.173 115.57) (end 114.808 114.935) (width 0.1524) (layer "F.Cu") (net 34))
 (segment (start 102.3068 121.476294) (end 103.133094 120.65) (width 0.1524) (layer "F.Cu") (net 34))
 (segment (start 114.808 110.49) (end 113.538 109.22) (width 0.1524) (layer "F.Cu") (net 34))
 (segment (start 102.3068 110.2912) (end 100.838 111.76) (width 0.1524) (layer "F.Cu") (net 31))
 (segment (start 103.378 106.68) (end 102.3068 107.7512) (width 0.1524) (layer "F.Cu") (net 31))
 (segment (start 102.3068 107.7512) (end 102.3068 110.2912) (width 0.1524) (layer "F.Cu") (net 31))
 (segment (start 118.618 99.06) (end 121.158 99.06) (width 0.1524) (layer "B.Cu") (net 5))
 (segment (start 118.618 96.52) (end 121.158 96.52) (width 0.1524) (layer "B.Cu") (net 4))
 (segment (start 118.618 93.98) (end 121.158 93.98) (width 0.1524) (layer "B.Cu") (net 3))
 (segment (start 117.5468 92.5112) (end 102.3068 92.5112) (width 0.1524) (layer "B.Cu") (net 24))
 (segment (start 102.3068 92.5112) (end 100.838 93.98) (width 0.1524) (layer "B.Cu") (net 24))
 (segment (start 118.618 91.44) (end 117.5468 92.5112) (width 0.1524) (layer "B.Cu") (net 24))
 (segment (start 101.9592 108.0988) (end 100.838 109.22) (width 0.1524) (layer "F.Cu") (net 30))
 (segment (start 101.9592 105.5588) (end 101.9592 108.0988) (width 0.1524) (layer "F.Cu") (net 30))
 (segment (start 103.378 104.14) (end 101.9592 105.5588) (width 0.1524) (layer "F.Cu") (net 30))
 (segment (start 101.616702 102.87) (end 102.886702 101.6) (width 0.1524) (layer "F.Cu") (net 32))
 (segment (start 99.568 102.87) (end 98.933 103.505) (width 0.1524) (layer "F.Cu") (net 32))
 (segment (start 98.933 103.505) (end 98.933 112.395) (width 0.1524) (layer "F.Cu") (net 32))
 (segment (start 99.568 102.87) (end 101.616702 102.87) (width 0.1524) (layer "F.Cu") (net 32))
 (segment (start 102.886702 101.6) (end 103.378 101.6) (width 0.1524) (layer "F.Cu") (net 32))
 (segment (start 98.933 112.395) (end 100.838 114.3) (width 0.1524) (layer "F.Cu") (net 32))
 (segment (start 102.2568 100.1812) (end 99.568 100.1812) (width 0.1524) (layer "F.Cu") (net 33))
 (segment (start 99.568 100.1812) (end 98.298 101.4512) (width 0.1524) (layer "F.Cu") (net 33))
 (segment (start 98.298 114.3) (end 100.838 116.84) (width 0.1524) (layer "F.Cu") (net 33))
 (segment (start 103.378 99.06) (end 102.2568 100.1812) (width 0.1524) (layer "F.Cu") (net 33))
 (segment (start 98.298 101.4512) (end 98.298 114.3) (width 0.1524) (layer "F.Cu") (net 33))
 (segment (start 98.298 124.46) (end 100.838 124.46) (width 0.1524) (layer "F.Cu") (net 35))
 (segment (start 101.9592 97.9388) (end 100.373583 97.9388) (width 0.1524) (layer "F.Cu") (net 35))
 (segment (start 100.373583 97.9388) (end 97.028 101.284383) (width 0.1524) (layer "F.Cu") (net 35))
 (segment (start 97.028 101.284383) (end 97.028 123.19) (width 0.1524) (layer "F.Cu") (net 35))
 (segment (start 103.378 96.52) (end 101.9592 97.9388) (width 0.1524) (layer "F.Cu") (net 35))
 (segment (start 97.028 123.19) (end 98.298 124.46) (width 0.1524) (layer "F.Cu") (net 35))
 (segment (start 100.838 96.52) (end 98.298 96.52) (width 0.1524) (layer "B.Cu") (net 25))
 (segment (start 98.298 90.17) (end 117.348 90.17) (width 0.1524) (layer "B.Cu") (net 25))
 (segment (start 117.348 90.17) (end 118.618 88.9) (width 0.1524) (layer "B.Cu") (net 25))
 (segment (start 98.298 96.52) (end 98.298 90.17) (width 0.1524) (layer "B.Cu") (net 25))
 (segment (start 97.663 88.9) (end 97.663 99.06) (width 0.1524) (layer "B.Cu") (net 26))
 (segment (start 103.378 88.9) (end 97.663 88.9) (width 0.1524) (layer "B.Cu") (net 26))
 (segment (start 97.663 99.06) (end 100.838 99.06) (width 0.1524) (layer "B.Cu") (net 26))
 (segment (start 118.618 134.62) (end 121.158 134.62) (width 0.1524) (layer "B.Cu") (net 18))
 (segment (start 103.378 124.46) (end 104.648 125.73) (width 0.1524) (layer "B.Cu") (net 14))
 (segment (start 120.666702 124.46) (end 121.158 124.46) (width 0.1524) (layer "B.Cu") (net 14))
 (segment (start 119.396702 125.73) (end 120.666702 124.46) (width 0.1524) (layer "B.Cu") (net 14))
 (segment (start 104.648 125.73) (end 119.396702 125.73) (width 0.1524) (layer "B.Cu") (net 14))
 (segment (start 118.618 119.38) (end 121.158 119.38) (width 0.1524) (layer "B.Cu") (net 13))
 (segment (start 118.618 116.84) (end 121.158 116.84) (width 0.1524) (layer "B.Cu") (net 12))
 (segment (start 118.618 114.3) (end 121.158 114.3) (width 0.1524) (layer "B.Cu") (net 11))
 (segment (start 118.618 111.76) (end 121.158 111.76) (width 0.1524) (layer "B.Cu") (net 10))
 (segment (start 118.618 109.22) (end 121.158 109.22) (width 0.1524) (layer "B.Cu") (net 9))
 (segment (start 118.618 106.68) (end 121.158 106.68) (width 0.1524) (layer "B.Cu") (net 8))
 (segment (start 118.618 104.14) (end 121.158 104.14) (width 0.1524) (layer "B.Cu") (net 7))
 (segment (start 118.618 101.6) (end 121.158 101.6) (width 0.1524) (layer "B.Cu") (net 6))
 (segment (start 128.778 127) (end 128.778 142.24) (width 0.1524) (layer "B.Cu") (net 15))
 (segment (start 128.778 142.24) (end 121.158 142.24) (width 0.1524) (layer "B.Cu") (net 15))
 (segment (start 121.158 127) (end 128.778 127) (width 0.1524) (layer "B.Cu") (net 15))
 (segment (start 116.078 129.54) (end 118.618 129.54) (width 0.1524) (layer "B.Cu") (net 43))
 (segment (start 103.378 127) (end 105.918 124.46) (width 0.1524) (layer "F.Cu") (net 45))
 (segment (start 116.078 115.57) (end 116.078 111.76) (width 0.1524) (layer "F.Cu") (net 45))
 (segment (start 109.728 116.205) (end 115.443 116.205) (width 0.1524) (layer "F.Cu") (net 45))
 (segment (start 105.918 124.46) (end 105.918 120.015) (width 0.1524) (layer "F.Cu") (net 45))
 (segment (start 115.443 116.205) (end 116.078 115.57) (width 0.1524) (layer "F.Cu") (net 45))
 (segment (start 105.918 120.015) (end 109.728 116.205) (width 0.1524) (layer "F.Cu") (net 45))
 (segment (start 107.823 114.935) (end 113.538 114.935) (width 0.1524) (layer "F.Cu") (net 23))
 (segment (start 113.538 114.935) (end 113.538 111.76) (width 0.1524) (layer "F.Cu") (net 23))
 (segment (start 103.378 119.38) (end 107.823 114.935) (width 0.1524) (layer "F.Cu") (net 23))
 (segment (start 130.9666 88.519503) (end 128.459697 86.0126) (width 0.1524) (layer "B.Cu") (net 21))
 (segment (start 130.048 125.73) (end 130.9666 124.8114) (width 0.1524) (layer "B.Cu") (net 21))
 (segment (start 130.9666 124.8114) (end 130.9666 88.519503) (width 0.1524) (layer "B.Cu") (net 21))
 (segment (start 119.888 125.73) (end 118.618 127) (width 0.1524) (layer "B.Cu") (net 21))
 (segment (start 128.459697 86.0126) (end 121.158 86.0126) (width 0.1524) (layer "B.Cu") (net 21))
 (segment (start 130.048 125.73) (end 119.888 125.73) (width 0.1524) (layer "B.Cu") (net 21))
 (segment (start 129.9842 88.9) (end 130.6192 89.535) (width 0.1524) (layer "B.Cu") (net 22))
 (segment (start 119.888 123.19) (end 128.778 123.19) (width 0.1524) (layer "B.Cu") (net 22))
 (segment (start 130.6192 121.3488) (end 130.6192 89.535) (width 0.1524) (layer "B.Cu") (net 22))
 (segment (start 121.158 88.9) (end 129.9842 88.9) (width 0.1524) (layer "B.Cu") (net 22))
 (segment (start 128.778 123.19) (end 130.6192 121.3488) (width 0.1524) (layer "B.Cu") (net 22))
 (segment (start 118.618 124.46) (end 119.888 123.19) (width 0.1524) (layer "B.Cu") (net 22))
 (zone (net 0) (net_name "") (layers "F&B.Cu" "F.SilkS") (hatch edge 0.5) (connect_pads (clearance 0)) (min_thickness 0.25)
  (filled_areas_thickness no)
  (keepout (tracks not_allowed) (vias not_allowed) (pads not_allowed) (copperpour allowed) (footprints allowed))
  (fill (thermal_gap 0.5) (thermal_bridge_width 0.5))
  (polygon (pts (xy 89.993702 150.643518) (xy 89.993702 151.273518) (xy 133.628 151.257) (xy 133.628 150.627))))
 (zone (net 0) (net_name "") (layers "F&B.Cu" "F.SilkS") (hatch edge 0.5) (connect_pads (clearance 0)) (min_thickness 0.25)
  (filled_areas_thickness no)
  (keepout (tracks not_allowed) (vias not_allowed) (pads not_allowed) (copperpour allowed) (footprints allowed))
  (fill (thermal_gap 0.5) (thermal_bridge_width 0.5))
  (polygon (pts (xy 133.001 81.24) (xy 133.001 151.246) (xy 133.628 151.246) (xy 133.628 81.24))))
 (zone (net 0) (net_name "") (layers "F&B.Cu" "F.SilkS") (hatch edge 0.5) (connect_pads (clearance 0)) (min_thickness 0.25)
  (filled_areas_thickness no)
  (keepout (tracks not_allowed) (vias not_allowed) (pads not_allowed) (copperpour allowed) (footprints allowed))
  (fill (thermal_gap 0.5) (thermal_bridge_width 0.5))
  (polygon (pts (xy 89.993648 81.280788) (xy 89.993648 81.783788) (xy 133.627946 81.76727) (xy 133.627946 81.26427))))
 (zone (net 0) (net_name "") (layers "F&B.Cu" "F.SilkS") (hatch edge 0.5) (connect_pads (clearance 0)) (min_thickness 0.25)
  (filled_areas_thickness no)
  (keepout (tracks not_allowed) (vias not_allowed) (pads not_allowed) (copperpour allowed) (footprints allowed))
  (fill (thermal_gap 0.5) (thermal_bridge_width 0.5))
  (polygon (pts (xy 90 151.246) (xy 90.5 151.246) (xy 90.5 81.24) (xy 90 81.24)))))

